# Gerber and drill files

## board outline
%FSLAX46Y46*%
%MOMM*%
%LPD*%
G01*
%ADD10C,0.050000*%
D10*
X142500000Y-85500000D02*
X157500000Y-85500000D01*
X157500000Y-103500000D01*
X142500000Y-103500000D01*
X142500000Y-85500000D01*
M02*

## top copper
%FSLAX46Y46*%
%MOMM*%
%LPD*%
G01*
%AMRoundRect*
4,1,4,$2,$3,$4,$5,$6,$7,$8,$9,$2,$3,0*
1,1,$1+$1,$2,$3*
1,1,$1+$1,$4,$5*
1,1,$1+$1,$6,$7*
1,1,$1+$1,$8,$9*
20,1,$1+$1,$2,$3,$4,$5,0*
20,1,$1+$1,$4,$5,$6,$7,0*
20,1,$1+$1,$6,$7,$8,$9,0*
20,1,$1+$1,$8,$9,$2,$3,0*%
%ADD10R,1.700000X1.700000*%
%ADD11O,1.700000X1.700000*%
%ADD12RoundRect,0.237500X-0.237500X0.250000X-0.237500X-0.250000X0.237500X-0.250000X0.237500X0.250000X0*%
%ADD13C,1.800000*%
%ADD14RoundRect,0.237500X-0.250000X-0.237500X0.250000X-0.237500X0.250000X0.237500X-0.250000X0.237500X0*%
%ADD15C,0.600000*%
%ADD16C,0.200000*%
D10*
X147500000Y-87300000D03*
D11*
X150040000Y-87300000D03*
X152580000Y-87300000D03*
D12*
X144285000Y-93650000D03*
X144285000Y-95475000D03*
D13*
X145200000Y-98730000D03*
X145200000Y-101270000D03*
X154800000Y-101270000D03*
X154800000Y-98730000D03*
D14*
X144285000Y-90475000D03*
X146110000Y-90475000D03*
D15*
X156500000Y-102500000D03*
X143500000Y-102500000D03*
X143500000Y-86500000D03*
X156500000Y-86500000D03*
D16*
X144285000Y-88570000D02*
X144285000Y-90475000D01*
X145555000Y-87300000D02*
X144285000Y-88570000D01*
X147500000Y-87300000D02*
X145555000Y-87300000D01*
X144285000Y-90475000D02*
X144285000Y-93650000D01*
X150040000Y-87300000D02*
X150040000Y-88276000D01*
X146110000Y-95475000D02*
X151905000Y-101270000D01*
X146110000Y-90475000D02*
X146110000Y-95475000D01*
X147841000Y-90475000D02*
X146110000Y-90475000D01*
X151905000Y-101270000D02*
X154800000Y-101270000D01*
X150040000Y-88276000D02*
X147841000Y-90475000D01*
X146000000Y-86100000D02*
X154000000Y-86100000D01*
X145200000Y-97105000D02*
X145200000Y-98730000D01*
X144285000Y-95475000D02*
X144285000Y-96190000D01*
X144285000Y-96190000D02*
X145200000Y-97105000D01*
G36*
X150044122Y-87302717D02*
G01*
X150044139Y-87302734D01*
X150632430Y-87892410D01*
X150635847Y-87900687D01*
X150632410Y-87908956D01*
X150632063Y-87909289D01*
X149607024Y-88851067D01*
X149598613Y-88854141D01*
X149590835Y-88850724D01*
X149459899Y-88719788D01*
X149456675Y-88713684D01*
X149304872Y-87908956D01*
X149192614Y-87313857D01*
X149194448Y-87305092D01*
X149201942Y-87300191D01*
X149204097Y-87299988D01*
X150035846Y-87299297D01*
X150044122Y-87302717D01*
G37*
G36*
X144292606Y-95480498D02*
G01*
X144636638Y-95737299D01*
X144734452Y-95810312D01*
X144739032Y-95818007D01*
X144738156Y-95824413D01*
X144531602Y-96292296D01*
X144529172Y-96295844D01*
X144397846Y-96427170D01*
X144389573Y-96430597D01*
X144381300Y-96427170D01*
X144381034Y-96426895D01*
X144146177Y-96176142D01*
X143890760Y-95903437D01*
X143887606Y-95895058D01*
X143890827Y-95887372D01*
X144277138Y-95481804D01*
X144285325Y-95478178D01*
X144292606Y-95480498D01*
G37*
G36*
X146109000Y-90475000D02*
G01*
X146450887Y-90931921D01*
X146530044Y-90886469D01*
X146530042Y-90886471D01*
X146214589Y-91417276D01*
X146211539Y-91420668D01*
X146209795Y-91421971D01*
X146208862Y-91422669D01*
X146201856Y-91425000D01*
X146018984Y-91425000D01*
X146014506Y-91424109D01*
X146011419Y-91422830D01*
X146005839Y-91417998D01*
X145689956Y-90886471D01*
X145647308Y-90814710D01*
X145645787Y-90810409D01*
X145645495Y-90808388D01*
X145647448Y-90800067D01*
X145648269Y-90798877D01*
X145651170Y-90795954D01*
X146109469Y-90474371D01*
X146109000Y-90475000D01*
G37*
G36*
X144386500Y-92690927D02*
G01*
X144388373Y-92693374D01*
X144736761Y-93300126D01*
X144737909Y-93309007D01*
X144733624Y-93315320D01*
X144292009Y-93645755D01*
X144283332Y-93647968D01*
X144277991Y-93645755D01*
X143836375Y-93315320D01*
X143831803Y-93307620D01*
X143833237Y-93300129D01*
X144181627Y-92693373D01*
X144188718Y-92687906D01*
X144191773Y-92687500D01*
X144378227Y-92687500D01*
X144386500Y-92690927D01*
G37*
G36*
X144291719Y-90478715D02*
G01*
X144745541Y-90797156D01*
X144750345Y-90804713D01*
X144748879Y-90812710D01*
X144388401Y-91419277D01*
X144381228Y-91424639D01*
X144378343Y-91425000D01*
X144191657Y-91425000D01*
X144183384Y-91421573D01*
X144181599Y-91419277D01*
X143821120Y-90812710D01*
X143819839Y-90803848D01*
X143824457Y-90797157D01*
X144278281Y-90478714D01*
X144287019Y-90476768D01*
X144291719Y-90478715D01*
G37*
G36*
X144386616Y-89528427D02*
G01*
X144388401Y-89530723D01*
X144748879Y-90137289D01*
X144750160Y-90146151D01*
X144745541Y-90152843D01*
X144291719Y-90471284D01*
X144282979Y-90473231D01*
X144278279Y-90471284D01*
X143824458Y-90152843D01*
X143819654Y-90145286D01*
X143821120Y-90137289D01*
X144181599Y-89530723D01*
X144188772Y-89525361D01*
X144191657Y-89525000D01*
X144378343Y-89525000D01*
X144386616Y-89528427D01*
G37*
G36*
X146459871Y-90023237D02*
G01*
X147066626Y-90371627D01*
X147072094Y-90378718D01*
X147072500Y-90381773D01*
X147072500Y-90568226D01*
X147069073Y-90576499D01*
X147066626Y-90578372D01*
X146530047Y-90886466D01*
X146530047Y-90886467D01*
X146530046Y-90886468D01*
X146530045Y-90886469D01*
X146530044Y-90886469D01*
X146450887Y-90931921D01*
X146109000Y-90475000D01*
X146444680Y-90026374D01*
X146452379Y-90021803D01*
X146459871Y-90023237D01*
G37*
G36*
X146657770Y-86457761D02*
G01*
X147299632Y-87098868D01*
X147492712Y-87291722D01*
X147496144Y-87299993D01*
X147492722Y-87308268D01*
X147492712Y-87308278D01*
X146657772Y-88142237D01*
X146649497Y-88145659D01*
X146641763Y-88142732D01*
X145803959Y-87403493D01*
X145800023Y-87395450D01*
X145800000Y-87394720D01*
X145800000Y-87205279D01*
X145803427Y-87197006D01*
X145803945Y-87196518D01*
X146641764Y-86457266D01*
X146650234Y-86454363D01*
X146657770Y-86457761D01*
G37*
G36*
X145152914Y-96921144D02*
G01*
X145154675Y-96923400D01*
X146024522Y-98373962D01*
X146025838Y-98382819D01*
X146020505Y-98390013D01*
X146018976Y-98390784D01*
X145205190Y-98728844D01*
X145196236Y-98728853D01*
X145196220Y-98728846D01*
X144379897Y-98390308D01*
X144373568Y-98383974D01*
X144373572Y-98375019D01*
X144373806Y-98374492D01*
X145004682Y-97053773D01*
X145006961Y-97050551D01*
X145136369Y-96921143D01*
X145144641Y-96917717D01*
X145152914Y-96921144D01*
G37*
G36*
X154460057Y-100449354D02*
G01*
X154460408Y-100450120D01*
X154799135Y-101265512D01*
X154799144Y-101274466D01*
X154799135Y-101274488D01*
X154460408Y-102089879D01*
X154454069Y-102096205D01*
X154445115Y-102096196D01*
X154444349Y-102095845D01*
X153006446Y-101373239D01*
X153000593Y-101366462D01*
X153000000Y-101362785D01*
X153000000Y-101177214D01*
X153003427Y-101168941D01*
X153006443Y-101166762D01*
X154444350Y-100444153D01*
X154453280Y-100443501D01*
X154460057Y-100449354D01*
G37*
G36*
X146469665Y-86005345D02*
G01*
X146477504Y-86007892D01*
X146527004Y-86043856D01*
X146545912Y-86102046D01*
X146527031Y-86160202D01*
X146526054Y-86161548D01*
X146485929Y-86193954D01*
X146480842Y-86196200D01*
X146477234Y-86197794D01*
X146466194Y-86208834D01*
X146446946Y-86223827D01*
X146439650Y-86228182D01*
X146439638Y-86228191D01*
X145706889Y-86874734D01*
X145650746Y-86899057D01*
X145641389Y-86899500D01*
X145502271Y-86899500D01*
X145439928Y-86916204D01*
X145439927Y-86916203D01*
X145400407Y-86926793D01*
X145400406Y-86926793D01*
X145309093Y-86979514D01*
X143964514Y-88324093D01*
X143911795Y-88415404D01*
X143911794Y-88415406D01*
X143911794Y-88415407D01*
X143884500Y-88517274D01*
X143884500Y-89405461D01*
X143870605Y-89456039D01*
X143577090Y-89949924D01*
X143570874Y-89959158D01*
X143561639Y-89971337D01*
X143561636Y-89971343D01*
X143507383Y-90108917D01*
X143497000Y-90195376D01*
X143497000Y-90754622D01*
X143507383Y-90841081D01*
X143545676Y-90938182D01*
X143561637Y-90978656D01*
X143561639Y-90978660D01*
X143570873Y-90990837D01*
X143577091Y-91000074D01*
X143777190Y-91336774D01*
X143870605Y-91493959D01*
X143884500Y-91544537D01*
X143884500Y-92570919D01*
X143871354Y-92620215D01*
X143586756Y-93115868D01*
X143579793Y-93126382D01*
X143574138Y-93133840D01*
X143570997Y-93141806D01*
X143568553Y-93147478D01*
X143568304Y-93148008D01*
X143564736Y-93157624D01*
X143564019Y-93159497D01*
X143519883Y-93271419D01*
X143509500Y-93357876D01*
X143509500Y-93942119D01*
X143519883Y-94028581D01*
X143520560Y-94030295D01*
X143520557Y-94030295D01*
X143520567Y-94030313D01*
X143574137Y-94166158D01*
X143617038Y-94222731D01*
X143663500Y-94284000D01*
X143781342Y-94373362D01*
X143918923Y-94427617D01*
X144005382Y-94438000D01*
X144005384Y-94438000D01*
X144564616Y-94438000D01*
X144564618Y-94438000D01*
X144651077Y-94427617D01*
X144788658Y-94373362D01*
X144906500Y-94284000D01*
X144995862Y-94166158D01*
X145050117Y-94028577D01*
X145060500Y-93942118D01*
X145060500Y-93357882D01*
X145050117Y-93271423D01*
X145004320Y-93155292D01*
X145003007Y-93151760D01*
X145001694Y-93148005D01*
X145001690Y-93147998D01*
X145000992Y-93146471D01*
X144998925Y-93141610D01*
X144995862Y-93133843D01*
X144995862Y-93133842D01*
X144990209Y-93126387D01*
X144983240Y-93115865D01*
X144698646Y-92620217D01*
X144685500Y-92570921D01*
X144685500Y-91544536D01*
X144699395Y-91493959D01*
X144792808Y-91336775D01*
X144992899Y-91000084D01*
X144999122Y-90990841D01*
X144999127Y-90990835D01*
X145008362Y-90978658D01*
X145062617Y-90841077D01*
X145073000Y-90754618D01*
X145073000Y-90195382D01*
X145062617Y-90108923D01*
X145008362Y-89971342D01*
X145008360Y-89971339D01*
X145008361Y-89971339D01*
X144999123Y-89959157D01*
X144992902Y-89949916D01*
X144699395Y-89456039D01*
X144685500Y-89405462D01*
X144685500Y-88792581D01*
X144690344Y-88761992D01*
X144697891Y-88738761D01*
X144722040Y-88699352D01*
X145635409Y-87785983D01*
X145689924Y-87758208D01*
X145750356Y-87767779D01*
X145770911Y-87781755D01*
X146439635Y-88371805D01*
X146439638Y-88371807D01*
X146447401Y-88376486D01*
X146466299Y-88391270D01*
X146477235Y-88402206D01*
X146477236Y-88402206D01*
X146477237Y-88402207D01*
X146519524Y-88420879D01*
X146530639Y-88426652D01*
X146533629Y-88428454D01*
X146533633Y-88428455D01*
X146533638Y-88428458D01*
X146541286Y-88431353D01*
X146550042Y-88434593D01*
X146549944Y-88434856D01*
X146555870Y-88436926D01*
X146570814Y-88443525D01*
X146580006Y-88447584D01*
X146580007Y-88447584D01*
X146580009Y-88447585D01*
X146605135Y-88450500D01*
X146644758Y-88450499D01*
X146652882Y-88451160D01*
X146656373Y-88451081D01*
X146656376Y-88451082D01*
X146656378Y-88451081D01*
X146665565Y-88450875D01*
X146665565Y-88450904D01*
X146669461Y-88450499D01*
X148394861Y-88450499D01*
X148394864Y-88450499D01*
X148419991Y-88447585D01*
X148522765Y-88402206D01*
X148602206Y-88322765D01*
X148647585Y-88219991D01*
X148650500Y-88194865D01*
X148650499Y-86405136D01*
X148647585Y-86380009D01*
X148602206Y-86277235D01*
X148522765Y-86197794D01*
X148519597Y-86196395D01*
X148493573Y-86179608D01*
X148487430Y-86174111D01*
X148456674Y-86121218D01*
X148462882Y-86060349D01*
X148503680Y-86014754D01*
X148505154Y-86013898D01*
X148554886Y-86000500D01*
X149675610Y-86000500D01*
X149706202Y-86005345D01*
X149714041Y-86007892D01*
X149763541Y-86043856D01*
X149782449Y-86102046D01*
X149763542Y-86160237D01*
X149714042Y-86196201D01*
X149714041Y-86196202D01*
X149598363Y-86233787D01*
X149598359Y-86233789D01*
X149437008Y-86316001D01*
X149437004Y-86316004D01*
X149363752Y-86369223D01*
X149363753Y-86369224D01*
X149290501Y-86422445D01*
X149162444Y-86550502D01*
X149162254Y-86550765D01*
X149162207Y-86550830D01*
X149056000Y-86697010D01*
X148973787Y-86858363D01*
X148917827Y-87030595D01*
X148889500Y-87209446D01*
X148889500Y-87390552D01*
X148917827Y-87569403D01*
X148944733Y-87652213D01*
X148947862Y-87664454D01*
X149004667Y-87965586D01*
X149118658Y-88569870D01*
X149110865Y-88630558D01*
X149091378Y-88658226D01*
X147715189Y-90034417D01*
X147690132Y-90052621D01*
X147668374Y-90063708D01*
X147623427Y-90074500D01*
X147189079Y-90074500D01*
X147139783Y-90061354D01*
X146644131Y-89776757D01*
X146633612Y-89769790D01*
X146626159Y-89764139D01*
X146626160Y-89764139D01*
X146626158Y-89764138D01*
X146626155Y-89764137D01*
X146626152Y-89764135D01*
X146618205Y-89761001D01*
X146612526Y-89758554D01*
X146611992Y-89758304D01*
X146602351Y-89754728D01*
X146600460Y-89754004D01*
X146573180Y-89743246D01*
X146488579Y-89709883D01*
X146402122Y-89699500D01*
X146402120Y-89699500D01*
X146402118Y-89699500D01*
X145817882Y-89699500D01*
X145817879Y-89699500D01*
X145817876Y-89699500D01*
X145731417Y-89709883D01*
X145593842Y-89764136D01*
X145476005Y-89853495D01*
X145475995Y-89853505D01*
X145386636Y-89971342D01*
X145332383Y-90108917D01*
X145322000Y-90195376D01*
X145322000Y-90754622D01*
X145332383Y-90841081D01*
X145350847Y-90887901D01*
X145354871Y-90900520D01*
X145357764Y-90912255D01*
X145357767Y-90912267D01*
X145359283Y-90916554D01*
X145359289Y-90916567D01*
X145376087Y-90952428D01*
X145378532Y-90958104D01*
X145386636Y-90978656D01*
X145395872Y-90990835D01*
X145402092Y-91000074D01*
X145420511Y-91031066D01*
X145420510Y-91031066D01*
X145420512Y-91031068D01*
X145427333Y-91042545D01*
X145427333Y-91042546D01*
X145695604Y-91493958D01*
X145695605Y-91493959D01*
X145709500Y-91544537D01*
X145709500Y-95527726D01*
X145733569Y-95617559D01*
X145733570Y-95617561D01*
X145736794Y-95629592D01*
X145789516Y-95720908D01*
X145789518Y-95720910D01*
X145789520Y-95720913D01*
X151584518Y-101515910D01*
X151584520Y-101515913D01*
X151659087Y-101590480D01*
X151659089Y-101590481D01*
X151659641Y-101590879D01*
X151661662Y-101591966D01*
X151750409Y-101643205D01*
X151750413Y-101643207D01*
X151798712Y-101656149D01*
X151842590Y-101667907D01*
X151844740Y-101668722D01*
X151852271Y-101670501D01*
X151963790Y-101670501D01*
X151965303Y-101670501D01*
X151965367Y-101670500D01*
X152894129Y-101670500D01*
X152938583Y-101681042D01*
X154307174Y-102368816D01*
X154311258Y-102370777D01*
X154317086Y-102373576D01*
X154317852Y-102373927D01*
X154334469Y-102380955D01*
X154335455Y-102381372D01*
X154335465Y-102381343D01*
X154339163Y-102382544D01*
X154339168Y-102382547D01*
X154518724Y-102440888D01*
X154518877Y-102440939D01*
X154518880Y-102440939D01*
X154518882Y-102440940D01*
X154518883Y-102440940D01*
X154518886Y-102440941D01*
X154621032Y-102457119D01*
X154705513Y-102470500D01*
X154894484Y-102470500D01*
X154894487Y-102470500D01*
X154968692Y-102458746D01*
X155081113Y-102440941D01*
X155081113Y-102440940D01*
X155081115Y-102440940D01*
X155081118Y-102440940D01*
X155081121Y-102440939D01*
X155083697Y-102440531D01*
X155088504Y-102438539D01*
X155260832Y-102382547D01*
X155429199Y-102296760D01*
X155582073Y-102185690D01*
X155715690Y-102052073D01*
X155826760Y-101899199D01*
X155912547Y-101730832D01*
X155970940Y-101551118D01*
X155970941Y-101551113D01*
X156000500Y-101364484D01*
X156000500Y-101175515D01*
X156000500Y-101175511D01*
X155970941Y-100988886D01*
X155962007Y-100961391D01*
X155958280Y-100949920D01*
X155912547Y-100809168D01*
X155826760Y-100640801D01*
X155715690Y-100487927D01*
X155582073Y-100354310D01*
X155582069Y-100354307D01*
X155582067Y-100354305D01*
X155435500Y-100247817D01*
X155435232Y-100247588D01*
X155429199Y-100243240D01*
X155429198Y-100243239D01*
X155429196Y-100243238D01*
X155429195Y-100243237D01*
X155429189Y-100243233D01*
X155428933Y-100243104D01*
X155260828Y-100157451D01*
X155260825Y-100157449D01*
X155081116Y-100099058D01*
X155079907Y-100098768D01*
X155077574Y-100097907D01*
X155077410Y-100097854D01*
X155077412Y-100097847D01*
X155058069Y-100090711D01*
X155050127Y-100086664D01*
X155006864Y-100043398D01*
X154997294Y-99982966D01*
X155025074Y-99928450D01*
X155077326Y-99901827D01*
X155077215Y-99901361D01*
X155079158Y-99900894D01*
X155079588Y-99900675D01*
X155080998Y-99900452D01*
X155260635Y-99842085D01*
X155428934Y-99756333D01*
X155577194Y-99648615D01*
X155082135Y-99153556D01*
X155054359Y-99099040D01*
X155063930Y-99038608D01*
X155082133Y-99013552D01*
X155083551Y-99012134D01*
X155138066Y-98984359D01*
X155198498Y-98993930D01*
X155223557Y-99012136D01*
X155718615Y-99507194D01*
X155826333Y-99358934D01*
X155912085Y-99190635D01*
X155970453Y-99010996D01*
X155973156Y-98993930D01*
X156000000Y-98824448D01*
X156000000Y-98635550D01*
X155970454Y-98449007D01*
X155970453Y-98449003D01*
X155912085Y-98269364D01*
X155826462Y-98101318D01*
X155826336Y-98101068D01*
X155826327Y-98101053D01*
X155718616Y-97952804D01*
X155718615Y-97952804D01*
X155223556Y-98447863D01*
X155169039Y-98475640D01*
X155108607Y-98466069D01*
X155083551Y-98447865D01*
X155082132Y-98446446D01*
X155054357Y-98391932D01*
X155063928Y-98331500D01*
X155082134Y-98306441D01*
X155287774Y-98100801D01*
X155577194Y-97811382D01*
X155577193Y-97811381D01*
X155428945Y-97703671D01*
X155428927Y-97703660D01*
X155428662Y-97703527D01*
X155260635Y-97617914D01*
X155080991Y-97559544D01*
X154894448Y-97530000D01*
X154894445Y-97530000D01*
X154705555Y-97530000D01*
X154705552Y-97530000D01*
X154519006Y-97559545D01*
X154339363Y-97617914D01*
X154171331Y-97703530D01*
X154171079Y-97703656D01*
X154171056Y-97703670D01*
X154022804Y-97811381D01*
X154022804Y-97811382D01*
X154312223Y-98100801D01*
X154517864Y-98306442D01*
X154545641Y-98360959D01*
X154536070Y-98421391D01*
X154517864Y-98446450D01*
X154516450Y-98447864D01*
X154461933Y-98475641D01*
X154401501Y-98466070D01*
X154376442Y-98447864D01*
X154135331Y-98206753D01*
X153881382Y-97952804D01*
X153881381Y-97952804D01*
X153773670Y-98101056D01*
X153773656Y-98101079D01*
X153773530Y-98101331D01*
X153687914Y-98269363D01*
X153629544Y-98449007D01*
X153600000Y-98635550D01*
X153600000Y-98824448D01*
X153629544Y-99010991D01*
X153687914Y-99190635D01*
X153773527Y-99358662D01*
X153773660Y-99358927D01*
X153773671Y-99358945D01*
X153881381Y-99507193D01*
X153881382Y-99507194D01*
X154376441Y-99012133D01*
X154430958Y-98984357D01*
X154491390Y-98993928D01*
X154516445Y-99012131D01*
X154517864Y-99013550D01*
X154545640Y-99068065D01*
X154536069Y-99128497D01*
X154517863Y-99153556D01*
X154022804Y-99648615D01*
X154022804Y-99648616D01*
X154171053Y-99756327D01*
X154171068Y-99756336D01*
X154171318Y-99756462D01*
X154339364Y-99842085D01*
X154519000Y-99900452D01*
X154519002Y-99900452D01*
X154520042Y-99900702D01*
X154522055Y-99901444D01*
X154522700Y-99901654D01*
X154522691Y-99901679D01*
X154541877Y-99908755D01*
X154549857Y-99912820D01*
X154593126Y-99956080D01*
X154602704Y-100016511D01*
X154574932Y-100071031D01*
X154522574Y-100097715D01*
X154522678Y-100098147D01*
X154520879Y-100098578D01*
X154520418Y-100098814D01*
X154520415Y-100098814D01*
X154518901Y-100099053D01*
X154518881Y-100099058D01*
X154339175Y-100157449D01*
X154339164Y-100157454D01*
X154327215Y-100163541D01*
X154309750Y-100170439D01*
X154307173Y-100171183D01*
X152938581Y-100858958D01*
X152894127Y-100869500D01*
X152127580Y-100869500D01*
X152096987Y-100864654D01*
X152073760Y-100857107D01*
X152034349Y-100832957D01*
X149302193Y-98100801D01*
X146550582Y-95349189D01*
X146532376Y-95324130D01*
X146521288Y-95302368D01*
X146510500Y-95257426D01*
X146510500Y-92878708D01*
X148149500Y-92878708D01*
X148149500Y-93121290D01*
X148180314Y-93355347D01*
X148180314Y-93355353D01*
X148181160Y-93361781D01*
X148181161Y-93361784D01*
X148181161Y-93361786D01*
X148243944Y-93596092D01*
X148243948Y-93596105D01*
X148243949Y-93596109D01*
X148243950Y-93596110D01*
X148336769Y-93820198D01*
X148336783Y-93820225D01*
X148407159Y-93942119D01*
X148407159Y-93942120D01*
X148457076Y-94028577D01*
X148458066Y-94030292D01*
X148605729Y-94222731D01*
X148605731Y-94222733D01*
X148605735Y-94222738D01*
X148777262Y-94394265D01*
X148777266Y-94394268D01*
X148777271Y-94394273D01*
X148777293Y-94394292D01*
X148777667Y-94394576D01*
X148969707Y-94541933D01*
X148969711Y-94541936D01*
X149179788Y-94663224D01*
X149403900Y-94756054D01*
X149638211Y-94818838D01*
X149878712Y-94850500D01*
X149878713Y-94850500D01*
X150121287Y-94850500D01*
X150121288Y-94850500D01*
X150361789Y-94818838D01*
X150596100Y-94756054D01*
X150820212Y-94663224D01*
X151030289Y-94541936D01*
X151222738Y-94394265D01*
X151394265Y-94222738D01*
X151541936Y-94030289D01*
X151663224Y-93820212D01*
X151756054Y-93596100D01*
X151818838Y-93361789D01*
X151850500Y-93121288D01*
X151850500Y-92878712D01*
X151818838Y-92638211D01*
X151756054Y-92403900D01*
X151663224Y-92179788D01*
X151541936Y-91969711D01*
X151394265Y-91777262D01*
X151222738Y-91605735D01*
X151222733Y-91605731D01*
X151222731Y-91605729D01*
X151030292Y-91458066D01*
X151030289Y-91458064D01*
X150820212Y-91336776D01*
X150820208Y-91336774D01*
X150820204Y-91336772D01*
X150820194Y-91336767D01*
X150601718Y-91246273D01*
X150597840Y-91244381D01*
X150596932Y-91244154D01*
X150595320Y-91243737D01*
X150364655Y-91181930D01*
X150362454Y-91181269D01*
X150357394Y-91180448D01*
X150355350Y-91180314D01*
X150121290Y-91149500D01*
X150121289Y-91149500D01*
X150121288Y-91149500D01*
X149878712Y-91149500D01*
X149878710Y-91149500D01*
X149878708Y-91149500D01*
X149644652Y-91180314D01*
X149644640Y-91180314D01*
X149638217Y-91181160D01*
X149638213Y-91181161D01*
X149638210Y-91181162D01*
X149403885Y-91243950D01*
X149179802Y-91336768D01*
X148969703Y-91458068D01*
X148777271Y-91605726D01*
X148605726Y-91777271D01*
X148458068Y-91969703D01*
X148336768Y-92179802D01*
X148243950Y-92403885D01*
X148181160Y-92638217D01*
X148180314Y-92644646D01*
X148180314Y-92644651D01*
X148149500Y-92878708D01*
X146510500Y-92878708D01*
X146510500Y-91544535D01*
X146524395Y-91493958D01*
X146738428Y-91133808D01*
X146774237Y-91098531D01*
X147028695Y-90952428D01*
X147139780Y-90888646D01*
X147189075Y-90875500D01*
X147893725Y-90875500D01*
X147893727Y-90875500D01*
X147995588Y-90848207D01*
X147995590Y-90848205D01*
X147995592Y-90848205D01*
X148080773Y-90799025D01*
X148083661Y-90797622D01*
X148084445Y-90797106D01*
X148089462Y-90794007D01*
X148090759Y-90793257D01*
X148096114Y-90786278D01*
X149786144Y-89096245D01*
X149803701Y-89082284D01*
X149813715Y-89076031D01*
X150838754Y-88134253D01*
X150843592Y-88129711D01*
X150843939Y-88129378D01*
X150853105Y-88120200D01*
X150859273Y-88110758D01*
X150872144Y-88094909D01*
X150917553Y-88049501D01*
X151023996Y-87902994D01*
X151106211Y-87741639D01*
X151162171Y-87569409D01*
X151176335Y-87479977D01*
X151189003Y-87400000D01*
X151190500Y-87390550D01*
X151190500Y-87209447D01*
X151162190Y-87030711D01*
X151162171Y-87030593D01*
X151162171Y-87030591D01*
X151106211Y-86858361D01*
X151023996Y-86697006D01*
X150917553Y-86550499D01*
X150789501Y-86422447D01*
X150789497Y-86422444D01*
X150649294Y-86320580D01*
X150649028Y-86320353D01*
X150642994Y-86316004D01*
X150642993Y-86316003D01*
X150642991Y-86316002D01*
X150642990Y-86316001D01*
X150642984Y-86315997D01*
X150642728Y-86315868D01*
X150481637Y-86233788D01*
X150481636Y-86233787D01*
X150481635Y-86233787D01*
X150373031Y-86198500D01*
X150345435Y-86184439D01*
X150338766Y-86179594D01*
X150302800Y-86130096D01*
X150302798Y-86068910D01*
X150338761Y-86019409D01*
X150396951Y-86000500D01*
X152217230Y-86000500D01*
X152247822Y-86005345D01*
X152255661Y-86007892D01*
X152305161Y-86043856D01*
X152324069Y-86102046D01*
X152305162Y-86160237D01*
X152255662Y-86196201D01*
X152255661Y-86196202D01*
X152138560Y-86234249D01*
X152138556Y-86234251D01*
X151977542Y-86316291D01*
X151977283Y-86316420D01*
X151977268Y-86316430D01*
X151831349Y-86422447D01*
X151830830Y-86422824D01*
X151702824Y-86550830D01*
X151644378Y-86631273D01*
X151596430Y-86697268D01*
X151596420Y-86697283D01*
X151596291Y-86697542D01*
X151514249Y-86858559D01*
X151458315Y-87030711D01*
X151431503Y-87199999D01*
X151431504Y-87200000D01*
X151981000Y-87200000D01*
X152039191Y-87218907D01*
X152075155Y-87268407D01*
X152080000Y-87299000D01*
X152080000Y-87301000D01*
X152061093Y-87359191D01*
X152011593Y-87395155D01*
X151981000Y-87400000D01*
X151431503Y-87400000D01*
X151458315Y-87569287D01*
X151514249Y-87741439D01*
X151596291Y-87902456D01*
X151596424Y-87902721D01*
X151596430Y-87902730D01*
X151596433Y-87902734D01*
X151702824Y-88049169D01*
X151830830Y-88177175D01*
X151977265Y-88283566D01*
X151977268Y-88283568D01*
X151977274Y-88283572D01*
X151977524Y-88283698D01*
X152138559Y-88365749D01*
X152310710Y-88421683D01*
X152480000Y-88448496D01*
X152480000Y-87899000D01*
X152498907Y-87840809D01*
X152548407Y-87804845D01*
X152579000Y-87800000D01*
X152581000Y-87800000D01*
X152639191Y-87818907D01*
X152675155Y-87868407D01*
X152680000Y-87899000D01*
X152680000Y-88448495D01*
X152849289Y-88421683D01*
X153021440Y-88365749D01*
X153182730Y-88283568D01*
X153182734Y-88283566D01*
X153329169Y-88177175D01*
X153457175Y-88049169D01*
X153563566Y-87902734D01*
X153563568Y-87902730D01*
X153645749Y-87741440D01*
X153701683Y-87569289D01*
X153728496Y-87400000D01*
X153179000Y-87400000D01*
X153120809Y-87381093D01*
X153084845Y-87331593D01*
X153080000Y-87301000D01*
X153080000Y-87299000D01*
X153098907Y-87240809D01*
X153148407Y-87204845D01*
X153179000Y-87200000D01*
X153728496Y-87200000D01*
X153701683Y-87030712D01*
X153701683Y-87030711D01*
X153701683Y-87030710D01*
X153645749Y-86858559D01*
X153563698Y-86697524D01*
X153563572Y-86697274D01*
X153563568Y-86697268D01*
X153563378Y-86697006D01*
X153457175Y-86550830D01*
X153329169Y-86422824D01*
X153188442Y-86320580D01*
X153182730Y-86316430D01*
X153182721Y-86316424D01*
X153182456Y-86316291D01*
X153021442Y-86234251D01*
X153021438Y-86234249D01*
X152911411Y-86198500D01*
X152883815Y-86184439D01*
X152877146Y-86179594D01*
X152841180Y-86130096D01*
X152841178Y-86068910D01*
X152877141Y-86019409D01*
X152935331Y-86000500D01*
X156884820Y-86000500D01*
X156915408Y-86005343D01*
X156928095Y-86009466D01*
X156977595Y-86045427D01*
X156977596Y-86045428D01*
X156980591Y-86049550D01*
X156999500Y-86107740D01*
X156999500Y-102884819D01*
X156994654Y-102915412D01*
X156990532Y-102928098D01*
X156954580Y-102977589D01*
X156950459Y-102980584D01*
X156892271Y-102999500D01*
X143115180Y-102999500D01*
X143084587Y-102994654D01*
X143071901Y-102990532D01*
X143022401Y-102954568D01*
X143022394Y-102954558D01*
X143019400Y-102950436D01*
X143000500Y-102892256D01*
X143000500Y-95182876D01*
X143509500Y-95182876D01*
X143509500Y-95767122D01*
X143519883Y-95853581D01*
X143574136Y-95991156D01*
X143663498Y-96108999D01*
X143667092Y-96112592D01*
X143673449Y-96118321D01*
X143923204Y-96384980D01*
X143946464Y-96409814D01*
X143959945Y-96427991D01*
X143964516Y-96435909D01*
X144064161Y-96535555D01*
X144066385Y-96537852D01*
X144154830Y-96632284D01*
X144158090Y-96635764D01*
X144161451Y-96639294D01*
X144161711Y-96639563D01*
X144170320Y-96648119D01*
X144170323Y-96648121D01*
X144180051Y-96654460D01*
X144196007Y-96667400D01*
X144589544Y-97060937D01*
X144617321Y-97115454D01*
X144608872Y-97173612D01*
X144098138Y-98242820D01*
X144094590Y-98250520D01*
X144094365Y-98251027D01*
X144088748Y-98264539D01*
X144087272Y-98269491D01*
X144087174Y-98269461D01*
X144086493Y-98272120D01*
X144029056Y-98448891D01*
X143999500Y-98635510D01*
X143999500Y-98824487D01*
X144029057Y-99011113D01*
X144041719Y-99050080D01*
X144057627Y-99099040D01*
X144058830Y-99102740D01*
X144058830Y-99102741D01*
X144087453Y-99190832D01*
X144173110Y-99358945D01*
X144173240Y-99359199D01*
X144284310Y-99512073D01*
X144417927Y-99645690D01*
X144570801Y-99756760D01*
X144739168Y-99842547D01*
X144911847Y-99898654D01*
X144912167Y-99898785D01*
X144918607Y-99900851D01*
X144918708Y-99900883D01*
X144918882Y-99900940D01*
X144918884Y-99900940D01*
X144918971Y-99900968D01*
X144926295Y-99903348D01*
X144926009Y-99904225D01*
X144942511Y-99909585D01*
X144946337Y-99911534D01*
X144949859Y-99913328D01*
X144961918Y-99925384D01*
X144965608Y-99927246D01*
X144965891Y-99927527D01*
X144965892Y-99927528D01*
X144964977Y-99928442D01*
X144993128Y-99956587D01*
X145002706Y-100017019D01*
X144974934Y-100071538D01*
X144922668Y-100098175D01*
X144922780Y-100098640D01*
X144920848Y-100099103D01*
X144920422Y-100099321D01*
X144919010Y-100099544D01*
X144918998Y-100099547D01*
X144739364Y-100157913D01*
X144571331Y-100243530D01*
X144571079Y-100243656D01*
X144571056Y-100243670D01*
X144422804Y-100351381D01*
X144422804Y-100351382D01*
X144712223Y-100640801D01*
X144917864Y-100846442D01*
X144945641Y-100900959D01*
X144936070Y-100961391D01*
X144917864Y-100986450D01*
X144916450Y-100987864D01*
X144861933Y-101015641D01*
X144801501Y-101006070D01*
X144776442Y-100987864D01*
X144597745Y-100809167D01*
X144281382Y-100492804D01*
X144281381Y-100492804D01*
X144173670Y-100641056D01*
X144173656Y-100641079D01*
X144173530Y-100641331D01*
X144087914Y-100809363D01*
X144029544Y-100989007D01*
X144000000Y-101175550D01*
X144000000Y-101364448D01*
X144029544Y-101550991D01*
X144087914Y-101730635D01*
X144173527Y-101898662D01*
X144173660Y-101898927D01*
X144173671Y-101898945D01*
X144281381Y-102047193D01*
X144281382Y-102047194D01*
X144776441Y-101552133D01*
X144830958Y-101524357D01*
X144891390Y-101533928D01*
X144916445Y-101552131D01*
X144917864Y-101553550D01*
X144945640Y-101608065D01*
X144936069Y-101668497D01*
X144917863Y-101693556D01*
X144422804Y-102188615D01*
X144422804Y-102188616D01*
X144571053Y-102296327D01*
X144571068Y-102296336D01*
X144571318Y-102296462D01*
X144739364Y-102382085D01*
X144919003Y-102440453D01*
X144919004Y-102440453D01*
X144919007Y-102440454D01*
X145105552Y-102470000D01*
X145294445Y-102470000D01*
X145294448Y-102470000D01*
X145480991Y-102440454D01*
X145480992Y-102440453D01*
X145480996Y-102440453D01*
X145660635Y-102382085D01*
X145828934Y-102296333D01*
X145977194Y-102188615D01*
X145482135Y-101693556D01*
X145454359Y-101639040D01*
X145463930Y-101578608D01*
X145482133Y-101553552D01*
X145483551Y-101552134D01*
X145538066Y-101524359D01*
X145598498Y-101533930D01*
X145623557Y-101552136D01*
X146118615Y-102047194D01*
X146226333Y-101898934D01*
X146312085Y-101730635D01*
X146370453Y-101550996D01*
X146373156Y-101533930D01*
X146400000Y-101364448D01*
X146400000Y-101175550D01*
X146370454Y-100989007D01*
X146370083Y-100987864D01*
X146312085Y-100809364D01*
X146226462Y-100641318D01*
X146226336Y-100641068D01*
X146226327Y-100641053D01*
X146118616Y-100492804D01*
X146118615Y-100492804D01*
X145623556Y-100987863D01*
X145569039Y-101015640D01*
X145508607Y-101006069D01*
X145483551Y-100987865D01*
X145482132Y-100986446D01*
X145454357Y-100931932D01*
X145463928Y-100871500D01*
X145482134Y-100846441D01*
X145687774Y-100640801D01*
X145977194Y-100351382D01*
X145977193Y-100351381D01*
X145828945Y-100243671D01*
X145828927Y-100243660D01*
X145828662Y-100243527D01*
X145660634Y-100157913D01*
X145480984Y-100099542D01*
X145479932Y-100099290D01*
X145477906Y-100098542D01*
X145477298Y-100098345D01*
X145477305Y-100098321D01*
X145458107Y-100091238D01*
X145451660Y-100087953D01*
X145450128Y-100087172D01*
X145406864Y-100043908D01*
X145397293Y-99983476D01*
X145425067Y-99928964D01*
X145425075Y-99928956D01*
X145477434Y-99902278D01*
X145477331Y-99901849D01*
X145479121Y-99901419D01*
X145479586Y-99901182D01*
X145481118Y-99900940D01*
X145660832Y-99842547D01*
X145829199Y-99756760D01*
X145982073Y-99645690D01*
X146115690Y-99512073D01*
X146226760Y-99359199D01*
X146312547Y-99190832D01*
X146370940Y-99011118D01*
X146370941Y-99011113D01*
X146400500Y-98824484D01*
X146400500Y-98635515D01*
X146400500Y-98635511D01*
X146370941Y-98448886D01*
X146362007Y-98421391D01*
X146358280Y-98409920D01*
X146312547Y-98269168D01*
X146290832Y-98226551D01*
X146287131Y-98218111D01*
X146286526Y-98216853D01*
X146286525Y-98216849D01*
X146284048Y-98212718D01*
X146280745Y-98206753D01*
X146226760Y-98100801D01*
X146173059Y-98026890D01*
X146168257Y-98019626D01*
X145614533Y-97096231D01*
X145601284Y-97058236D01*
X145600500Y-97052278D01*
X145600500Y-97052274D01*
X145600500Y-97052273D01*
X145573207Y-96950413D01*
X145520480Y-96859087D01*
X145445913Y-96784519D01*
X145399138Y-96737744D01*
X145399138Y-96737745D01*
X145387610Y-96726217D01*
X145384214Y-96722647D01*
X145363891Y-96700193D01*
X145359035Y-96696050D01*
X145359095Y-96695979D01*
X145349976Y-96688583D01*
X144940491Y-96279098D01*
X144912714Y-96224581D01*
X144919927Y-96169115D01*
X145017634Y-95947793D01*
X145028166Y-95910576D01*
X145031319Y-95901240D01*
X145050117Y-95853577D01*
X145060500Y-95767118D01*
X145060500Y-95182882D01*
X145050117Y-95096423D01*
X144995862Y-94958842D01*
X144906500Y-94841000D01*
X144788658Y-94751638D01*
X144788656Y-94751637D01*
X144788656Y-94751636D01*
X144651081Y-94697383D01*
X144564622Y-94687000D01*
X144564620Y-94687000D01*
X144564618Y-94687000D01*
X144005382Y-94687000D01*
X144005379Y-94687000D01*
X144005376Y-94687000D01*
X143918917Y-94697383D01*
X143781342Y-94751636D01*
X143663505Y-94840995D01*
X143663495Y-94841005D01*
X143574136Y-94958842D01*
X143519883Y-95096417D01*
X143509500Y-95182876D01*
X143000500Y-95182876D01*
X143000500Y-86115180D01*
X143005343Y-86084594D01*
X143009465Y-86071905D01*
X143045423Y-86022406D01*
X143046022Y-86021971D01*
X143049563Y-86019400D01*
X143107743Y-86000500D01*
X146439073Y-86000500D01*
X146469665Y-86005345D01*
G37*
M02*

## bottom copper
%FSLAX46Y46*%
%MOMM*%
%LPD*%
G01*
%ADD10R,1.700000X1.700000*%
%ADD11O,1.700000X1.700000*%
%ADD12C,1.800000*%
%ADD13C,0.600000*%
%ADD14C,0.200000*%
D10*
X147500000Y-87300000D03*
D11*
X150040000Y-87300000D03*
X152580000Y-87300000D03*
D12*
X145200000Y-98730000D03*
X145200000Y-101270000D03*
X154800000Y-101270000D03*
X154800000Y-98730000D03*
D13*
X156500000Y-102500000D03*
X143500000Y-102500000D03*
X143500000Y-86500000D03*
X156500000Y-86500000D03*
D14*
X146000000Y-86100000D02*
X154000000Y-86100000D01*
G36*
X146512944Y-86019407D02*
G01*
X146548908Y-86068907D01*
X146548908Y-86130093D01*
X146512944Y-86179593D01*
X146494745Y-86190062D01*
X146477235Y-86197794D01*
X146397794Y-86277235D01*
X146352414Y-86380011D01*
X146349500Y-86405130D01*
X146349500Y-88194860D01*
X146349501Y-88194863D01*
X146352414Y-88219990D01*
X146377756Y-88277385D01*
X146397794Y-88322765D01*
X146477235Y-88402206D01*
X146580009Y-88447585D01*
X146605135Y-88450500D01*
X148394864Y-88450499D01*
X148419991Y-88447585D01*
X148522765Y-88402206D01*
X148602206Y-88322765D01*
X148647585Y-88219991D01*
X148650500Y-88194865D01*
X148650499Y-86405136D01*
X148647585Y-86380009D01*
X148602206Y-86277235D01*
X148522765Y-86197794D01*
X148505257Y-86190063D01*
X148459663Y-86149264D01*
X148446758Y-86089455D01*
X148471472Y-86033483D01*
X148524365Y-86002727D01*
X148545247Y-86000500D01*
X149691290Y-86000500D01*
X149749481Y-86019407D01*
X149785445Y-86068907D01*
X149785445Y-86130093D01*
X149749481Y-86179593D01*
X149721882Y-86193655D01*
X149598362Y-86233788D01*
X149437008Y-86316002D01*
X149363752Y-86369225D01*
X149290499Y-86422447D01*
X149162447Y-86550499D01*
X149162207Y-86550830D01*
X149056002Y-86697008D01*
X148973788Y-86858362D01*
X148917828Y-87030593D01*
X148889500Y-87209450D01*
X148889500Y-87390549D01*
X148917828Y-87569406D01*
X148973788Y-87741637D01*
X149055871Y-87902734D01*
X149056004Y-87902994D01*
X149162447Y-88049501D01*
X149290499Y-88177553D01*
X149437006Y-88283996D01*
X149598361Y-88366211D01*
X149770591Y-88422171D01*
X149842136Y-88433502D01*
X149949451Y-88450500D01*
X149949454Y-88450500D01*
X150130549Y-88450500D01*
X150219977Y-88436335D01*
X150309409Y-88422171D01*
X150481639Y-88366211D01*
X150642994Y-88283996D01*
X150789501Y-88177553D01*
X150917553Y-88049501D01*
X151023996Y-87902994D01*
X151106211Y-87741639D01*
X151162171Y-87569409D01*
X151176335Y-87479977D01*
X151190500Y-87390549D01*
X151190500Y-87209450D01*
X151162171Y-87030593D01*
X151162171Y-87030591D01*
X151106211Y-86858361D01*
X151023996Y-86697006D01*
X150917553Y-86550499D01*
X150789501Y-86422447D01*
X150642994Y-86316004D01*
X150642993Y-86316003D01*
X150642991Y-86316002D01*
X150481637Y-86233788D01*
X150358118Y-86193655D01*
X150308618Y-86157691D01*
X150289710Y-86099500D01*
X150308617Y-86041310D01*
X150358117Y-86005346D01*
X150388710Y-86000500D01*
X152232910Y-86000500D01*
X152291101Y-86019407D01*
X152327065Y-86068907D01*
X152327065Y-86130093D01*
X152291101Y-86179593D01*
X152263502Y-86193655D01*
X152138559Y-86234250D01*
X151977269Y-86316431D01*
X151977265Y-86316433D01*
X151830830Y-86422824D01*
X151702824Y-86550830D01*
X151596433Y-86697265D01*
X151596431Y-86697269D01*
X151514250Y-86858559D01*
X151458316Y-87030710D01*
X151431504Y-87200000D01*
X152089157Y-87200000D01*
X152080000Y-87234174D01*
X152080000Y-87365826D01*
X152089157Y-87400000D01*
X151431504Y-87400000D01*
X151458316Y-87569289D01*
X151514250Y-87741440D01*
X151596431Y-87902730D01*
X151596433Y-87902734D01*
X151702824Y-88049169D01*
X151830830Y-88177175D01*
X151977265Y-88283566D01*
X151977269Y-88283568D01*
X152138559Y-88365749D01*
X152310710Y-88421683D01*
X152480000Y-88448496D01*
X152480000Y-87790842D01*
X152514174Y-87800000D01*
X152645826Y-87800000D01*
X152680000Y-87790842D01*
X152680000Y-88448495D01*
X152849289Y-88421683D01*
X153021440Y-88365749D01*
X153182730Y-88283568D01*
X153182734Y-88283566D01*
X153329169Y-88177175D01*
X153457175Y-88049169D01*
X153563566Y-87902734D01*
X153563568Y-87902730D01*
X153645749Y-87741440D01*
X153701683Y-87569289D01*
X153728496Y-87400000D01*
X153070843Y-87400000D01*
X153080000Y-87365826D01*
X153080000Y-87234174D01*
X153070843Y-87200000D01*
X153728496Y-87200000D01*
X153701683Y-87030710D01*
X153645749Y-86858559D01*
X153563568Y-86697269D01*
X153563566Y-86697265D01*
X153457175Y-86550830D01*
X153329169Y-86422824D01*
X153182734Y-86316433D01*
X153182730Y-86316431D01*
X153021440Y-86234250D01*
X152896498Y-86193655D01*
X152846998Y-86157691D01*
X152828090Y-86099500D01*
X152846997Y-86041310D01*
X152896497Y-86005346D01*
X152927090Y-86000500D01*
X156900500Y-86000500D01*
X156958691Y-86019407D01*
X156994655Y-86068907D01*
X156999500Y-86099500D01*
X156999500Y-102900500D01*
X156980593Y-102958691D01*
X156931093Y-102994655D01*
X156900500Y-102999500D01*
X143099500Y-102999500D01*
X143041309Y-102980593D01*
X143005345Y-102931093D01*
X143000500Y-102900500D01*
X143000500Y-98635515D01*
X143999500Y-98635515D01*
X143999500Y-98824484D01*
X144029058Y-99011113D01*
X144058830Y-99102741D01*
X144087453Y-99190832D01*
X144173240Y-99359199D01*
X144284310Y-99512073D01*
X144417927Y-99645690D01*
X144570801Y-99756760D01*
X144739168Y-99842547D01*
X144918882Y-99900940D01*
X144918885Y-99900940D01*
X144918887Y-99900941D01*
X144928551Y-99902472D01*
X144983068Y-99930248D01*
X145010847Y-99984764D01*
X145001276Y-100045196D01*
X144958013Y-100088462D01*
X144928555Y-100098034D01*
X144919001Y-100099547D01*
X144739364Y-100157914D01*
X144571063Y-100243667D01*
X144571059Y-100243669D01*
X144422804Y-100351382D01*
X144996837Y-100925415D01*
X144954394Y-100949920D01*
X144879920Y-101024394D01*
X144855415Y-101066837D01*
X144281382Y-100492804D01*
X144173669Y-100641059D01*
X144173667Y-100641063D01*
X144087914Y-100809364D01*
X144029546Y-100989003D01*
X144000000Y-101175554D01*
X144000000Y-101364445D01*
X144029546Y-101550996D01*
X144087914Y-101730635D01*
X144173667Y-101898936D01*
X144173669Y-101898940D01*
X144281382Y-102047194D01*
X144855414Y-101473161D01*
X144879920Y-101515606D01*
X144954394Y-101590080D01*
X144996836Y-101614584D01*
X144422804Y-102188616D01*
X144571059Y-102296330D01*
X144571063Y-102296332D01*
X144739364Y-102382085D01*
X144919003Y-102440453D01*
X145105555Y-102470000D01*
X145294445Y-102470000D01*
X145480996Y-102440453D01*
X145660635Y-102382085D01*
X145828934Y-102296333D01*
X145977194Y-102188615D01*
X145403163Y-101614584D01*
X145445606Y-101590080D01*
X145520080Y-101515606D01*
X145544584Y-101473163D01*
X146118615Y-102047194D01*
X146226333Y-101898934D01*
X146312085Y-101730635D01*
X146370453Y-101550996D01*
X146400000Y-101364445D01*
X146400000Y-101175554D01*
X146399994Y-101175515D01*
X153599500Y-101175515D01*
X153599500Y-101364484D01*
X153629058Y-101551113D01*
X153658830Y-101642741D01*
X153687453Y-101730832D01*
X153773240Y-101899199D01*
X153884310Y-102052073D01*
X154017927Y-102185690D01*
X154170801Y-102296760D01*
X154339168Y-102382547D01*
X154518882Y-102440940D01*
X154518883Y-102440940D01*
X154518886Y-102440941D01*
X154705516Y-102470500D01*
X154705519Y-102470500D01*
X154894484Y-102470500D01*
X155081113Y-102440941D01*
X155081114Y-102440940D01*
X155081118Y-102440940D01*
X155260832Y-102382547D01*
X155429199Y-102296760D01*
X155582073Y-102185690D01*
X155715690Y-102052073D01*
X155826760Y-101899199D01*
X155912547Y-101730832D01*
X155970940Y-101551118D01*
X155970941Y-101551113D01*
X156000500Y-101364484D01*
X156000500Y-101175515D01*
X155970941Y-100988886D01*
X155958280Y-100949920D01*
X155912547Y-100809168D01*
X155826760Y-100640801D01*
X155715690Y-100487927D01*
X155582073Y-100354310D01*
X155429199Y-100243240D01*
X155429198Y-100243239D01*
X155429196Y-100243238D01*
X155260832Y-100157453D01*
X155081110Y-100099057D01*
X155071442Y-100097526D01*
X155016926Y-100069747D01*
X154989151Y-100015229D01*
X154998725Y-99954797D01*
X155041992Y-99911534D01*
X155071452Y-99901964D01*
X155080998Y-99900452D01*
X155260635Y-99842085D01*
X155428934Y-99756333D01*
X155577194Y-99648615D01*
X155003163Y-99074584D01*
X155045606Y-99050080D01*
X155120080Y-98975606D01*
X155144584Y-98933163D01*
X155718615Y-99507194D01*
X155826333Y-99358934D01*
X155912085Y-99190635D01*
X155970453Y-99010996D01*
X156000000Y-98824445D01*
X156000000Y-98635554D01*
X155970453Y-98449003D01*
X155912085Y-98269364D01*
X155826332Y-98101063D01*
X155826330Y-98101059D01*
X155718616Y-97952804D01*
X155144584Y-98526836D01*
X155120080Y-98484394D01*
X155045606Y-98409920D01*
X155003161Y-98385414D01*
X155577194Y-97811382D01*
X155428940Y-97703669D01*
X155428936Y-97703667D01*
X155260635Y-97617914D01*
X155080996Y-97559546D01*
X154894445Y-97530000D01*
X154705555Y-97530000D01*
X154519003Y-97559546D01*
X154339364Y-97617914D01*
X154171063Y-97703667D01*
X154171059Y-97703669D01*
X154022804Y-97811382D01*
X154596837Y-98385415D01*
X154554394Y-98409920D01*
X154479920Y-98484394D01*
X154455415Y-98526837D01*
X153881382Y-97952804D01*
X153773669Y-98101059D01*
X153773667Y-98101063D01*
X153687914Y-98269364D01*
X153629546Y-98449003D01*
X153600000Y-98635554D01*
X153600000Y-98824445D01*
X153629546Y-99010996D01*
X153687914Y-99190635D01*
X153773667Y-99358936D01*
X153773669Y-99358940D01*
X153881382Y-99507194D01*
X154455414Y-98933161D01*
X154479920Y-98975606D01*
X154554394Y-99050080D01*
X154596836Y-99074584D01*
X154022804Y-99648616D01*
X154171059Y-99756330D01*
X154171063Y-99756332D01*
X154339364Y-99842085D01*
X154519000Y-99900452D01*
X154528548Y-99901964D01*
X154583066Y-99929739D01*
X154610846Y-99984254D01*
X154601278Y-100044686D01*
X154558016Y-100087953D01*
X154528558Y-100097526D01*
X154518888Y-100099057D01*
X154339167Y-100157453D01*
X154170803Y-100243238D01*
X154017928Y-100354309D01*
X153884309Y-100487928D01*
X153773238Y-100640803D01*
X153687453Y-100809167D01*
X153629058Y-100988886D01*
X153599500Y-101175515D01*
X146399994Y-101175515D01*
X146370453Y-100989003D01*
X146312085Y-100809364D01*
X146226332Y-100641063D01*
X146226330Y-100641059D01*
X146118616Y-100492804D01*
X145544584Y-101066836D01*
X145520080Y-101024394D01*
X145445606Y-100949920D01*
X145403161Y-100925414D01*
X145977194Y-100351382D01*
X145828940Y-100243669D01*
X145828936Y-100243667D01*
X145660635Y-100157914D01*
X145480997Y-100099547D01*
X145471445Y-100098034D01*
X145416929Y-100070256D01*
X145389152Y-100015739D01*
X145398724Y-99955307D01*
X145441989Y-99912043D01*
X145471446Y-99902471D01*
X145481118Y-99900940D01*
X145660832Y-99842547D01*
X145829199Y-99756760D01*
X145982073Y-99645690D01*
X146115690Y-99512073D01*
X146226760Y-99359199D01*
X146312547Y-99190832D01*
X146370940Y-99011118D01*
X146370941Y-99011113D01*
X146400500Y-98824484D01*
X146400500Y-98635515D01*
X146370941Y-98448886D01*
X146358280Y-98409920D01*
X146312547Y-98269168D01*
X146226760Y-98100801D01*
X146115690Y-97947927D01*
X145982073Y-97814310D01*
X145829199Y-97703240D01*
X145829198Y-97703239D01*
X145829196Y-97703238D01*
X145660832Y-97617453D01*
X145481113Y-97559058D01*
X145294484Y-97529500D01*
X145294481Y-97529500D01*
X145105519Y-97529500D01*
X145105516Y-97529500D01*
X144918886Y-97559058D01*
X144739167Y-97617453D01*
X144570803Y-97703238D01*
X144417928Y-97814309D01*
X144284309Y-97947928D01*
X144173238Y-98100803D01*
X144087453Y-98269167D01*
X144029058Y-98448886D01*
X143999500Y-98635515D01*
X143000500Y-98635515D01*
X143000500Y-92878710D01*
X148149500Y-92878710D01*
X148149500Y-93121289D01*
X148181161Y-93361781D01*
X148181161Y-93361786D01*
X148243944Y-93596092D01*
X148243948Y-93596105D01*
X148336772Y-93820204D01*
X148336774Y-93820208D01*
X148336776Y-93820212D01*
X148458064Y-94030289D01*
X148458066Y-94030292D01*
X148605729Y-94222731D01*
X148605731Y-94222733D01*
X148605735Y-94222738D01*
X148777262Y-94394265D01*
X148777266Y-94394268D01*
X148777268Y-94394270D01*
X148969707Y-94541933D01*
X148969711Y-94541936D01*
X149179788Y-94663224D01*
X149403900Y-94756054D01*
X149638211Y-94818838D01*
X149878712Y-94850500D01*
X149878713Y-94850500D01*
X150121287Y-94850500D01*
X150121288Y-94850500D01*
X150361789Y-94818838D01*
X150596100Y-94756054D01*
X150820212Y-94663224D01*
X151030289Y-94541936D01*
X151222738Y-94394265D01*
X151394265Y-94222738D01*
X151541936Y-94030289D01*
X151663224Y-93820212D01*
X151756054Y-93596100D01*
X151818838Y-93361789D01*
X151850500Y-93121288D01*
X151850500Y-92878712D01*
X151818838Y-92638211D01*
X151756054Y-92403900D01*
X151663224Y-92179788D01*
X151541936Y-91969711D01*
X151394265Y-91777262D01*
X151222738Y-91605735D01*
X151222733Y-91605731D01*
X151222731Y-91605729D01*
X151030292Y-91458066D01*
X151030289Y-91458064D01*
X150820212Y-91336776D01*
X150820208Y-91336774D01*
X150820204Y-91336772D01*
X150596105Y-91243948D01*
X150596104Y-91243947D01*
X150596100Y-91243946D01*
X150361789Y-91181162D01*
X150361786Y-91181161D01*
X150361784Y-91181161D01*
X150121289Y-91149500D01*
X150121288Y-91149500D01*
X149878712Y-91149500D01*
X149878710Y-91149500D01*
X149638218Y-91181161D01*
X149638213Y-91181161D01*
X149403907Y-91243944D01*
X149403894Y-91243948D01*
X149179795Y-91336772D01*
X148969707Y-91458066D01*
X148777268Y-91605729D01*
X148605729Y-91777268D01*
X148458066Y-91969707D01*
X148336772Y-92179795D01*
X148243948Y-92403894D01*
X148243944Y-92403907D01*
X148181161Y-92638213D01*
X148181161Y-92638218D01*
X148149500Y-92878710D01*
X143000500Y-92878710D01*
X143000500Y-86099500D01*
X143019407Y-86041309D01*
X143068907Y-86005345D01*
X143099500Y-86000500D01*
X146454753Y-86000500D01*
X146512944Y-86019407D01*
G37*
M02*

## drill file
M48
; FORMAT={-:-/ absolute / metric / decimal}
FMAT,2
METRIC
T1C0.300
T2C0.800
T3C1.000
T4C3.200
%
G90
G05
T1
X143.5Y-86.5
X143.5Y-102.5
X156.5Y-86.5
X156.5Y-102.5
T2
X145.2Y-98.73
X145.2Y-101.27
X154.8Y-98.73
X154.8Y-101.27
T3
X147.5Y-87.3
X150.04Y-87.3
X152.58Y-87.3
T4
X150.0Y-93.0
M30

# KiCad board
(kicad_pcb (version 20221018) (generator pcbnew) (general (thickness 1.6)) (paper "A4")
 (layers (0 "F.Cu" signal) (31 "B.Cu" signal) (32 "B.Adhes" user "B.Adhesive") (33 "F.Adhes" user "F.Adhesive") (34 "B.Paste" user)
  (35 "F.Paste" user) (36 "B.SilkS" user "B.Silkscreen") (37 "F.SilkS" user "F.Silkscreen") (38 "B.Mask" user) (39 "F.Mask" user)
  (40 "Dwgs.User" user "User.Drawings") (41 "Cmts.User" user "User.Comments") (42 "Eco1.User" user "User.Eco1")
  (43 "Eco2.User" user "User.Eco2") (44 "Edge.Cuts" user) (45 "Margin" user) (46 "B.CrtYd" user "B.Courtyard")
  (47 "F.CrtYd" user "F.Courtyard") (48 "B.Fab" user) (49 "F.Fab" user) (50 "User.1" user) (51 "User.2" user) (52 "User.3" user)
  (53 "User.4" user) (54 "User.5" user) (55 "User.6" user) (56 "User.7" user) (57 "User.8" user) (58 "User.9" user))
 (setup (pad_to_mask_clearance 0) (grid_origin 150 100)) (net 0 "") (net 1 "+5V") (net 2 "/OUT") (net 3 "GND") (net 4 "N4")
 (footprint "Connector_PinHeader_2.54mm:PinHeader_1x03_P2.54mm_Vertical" (layer "F.Cu") (at 147.5 87.3 90)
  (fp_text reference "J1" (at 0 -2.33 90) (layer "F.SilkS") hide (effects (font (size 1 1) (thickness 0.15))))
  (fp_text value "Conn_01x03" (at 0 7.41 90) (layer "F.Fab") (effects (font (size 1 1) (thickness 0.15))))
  (pad "1" thru_hole rect (at 0 0 90) (size 1.7 1.7) (drill 1) (layers "*.Cu" "*.Mask") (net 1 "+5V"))
  (pad "2" thru_hole oval (at 0 2.54 90) (size 1.7 1.7) (drill 1) (layers "*.Cu" "*.Mask") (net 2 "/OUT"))
  (pad "3" thru_hole oval (at 0 5.08 90) (size 1.7 1.7) (drill 1) (layers "*.Cu" "*.Mask") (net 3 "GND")))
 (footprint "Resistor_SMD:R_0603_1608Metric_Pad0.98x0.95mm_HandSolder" (layer "F.Cu") (at 144.285 94.5625 -90)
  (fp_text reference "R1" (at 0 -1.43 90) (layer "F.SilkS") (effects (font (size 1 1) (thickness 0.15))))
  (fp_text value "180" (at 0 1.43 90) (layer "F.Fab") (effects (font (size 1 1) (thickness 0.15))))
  (pad "1" smd roundrect (at -0.9125 0 270) (size 0.975 0.95) (layers "F.Cu" "F.Paste" "F.Mask") (roundrect_rratio 0.25) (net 1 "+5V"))
  (pad "2" smd roundrect (at 0.9125 0 270) (size 0.975 0.95) (layers "F.Cu" "F.Paste" "F.Mask") (roundrect_rratio 0.25) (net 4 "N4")))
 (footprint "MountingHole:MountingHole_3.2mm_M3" (layer "F.Cu") (at 150 93)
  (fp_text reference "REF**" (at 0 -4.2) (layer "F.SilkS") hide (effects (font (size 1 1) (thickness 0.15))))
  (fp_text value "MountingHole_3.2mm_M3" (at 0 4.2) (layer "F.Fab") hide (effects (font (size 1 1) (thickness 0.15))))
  (pad "" np_thru_hole circle (at 0 0) (size 3.2 3.2) (drill 3.2) (layers "*.Cu" "*.Mask")))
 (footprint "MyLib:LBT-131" (layer "F.Cu") (at 150 100)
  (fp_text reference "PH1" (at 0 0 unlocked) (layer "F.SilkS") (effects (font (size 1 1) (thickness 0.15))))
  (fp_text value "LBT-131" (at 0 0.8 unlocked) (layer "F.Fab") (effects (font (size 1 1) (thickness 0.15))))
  (pad "1" thru_hole circle (at -4.8 -1.27) (size 1.8 1.8) (drill 0.8) (layers "*.Cu" "*.Mask") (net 4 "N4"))
  (pad "2" thru_hole circle (at -4.8 1.27) (size 1.8 1.8) (drill 0.8) (layers "*.Cu" "*.Mask") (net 3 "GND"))
  (pad "3" thru_hole circle (at 4.8 1.27) (size 1.8 1.8) (drill 0.8) (layers "*.Cu" "*.Mask") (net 2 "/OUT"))
  (pad "4" thru_hole circle (at 4.8 -1.27) (size 1.8 1.8) (drill 0.8) (layers "*.Cu" "*.Mask") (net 3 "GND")))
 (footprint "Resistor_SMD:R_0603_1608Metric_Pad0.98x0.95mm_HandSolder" (layer "F.Cu") (at 145.1975 90.475)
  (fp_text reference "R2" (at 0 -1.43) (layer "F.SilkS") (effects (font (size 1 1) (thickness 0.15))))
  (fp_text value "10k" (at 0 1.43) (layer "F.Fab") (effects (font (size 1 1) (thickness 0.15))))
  (pad "1" smd roundrect (at -0.9125 0) (size 0.975 0.95) (layers "F.Cu" "F.Paste" "F.Mask") (roundrect_rratio 0.25) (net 1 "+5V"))
  (pad "2" smd roundrect (at 0.9125 0) (size 0.975 0.95) (layers "F.Cu" "F.Paste" "F.Mask") (roundrect_rratio 0.25) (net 2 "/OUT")))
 (gr_rect (start 142.5 85.5) (end 157.5 103.5) (stroke (width 0.05) (type default)) (fill none) (layer "Edge.Cuts"))
 (segment (start 144.285 88.57) (end 144.285 90.475) (width 0.2) (layer "F.Cu") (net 1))
 (segment (start 145.555 87.3) (end 144.285 88.57) (width 0.2) (layer "F.Cu") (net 1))
 (segment (start 147.5 87.3) (end 145.555 87.3) (width 0.2) (layer "F.Cu") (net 1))
 (segment (start 144.285 90.475) (end 144.285 93.65) (width 0.2) (layer "F.Cu") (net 1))
 (segment (start 150.04 87.3) (end 150.04 88.276) (width 0.2) (layer "F.Cu") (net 2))
 (segment (start 146.11 95.475) (end 151.905 101.27) (width 0.2) (layer "F.Cu") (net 2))
 (segment (start 146.11 90.475) (end 146.11 95.475) (width 0.2) (layer "F.Cu") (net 2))
 (segment (start 147.841 90.475) (end 146.11 90.475) (width 0.2) (layer "F.Cu") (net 2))
 (segment (start 151.905 101.27) (end 154.8 101.27) (width 0.2) (layer "F.Cu") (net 2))
 (segment (start 150.04 88.276) (end 147.841 90.475) (width 0.2) (layer "F.Cu") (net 2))
 (segment (start 146 86.1) (end 154 86.1) (width 0.2) (layer "F.Cu") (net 3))
 (via (at 156.5 102.5) (size 0.6) (drill 0.3) (layers "F.Cu" "B.Cu") (free) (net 3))
 (via (at 143.5 102.5) (size 0.6) (drill 0.3) (layers "F.Cu" "B.Cu") (free) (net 3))
 (via (at 143.5 86.5) (size 0.6) (drill 0.3) (layers "F.Cu" "B.Cu") (free) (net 3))
 (via (at 156.5 86.5) (size 0.6) (drill 0.3) (layers "F.Cu" "B.Cu") (free) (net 3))
 (segment (start 146 86.1) (end 154 86.1) (width 0.2) (layer "B.Cu") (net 3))
 (segment (start 145.2 97.105) (end 145.2 98.73) (width 0.2) (layer "F.Cu") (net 4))
 (segment (start 144.285 95.475) (end 144.285 96.19) (width 0.2) (layer "F.Cu") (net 4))
 (segment (start 144.285 96.19) (end 145.2 97.105) (width 0.2) (layer "F.Cu") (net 4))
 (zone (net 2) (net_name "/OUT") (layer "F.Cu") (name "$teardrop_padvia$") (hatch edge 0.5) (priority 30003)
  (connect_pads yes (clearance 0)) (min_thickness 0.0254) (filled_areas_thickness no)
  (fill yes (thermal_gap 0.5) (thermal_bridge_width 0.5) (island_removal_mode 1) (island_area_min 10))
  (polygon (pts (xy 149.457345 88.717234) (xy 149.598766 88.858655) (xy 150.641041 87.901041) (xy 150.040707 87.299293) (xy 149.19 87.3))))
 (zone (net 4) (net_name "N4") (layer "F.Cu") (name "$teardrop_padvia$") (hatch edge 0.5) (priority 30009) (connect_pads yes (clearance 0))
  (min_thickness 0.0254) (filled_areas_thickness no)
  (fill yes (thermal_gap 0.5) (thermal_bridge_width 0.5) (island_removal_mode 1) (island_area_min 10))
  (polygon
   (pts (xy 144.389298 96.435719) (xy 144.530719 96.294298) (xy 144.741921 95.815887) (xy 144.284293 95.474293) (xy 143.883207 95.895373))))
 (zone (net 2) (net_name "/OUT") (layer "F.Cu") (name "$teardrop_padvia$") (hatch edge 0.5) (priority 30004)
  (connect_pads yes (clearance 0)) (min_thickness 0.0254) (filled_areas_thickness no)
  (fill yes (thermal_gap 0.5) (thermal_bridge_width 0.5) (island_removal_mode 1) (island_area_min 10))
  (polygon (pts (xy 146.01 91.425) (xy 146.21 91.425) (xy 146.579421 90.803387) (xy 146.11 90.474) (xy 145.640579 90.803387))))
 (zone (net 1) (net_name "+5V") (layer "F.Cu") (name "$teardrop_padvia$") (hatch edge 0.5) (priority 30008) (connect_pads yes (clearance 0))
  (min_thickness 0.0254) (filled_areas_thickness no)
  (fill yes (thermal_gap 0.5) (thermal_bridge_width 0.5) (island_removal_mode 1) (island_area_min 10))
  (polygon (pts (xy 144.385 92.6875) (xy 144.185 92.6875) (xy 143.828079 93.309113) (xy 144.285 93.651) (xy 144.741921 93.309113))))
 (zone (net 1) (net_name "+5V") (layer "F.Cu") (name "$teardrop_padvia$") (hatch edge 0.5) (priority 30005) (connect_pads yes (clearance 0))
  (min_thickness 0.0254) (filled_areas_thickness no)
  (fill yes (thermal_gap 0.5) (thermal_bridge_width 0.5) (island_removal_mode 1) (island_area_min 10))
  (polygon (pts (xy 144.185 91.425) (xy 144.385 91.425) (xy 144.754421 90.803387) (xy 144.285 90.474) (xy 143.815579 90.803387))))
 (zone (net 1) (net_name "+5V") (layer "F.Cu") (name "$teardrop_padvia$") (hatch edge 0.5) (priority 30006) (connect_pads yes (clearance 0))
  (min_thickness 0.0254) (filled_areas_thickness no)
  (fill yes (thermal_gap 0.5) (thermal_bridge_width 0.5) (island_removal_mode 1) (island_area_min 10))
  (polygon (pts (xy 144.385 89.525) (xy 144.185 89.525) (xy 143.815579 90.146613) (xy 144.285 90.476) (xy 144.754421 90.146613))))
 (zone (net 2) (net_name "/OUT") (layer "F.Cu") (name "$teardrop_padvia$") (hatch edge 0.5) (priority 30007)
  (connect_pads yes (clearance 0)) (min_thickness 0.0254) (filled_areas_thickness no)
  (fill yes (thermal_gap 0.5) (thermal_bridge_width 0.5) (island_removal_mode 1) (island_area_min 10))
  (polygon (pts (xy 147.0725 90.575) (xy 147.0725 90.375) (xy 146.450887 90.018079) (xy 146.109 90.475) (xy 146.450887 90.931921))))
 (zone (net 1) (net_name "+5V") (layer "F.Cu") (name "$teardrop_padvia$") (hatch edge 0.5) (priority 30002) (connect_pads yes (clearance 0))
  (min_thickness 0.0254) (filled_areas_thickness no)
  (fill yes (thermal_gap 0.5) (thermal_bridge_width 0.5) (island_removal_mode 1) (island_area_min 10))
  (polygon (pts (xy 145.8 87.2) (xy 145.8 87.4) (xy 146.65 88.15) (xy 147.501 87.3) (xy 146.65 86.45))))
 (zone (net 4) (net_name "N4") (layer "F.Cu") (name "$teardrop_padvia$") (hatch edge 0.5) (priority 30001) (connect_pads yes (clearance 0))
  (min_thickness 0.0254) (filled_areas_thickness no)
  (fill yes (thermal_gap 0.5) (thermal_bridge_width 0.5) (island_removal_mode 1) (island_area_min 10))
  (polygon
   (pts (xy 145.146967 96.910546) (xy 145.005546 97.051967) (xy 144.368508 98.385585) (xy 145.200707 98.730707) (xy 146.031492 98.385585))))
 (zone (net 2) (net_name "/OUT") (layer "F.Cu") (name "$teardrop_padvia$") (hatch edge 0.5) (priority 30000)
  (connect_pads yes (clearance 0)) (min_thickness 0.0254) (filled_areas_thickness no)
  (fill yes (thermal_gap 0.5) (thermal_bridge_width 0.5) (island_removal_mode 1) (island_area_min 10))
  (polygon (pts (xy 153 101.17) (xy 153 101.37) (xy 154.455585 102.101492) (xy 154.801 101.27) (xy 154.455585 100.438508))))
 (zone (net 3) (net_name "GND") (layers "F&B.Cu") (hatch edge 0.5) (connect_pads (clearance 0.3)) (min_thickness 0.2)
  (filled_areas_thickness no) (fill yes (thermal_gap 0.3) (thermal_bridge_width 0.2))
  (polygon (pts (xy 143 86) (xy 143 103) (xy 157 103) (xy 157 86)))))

